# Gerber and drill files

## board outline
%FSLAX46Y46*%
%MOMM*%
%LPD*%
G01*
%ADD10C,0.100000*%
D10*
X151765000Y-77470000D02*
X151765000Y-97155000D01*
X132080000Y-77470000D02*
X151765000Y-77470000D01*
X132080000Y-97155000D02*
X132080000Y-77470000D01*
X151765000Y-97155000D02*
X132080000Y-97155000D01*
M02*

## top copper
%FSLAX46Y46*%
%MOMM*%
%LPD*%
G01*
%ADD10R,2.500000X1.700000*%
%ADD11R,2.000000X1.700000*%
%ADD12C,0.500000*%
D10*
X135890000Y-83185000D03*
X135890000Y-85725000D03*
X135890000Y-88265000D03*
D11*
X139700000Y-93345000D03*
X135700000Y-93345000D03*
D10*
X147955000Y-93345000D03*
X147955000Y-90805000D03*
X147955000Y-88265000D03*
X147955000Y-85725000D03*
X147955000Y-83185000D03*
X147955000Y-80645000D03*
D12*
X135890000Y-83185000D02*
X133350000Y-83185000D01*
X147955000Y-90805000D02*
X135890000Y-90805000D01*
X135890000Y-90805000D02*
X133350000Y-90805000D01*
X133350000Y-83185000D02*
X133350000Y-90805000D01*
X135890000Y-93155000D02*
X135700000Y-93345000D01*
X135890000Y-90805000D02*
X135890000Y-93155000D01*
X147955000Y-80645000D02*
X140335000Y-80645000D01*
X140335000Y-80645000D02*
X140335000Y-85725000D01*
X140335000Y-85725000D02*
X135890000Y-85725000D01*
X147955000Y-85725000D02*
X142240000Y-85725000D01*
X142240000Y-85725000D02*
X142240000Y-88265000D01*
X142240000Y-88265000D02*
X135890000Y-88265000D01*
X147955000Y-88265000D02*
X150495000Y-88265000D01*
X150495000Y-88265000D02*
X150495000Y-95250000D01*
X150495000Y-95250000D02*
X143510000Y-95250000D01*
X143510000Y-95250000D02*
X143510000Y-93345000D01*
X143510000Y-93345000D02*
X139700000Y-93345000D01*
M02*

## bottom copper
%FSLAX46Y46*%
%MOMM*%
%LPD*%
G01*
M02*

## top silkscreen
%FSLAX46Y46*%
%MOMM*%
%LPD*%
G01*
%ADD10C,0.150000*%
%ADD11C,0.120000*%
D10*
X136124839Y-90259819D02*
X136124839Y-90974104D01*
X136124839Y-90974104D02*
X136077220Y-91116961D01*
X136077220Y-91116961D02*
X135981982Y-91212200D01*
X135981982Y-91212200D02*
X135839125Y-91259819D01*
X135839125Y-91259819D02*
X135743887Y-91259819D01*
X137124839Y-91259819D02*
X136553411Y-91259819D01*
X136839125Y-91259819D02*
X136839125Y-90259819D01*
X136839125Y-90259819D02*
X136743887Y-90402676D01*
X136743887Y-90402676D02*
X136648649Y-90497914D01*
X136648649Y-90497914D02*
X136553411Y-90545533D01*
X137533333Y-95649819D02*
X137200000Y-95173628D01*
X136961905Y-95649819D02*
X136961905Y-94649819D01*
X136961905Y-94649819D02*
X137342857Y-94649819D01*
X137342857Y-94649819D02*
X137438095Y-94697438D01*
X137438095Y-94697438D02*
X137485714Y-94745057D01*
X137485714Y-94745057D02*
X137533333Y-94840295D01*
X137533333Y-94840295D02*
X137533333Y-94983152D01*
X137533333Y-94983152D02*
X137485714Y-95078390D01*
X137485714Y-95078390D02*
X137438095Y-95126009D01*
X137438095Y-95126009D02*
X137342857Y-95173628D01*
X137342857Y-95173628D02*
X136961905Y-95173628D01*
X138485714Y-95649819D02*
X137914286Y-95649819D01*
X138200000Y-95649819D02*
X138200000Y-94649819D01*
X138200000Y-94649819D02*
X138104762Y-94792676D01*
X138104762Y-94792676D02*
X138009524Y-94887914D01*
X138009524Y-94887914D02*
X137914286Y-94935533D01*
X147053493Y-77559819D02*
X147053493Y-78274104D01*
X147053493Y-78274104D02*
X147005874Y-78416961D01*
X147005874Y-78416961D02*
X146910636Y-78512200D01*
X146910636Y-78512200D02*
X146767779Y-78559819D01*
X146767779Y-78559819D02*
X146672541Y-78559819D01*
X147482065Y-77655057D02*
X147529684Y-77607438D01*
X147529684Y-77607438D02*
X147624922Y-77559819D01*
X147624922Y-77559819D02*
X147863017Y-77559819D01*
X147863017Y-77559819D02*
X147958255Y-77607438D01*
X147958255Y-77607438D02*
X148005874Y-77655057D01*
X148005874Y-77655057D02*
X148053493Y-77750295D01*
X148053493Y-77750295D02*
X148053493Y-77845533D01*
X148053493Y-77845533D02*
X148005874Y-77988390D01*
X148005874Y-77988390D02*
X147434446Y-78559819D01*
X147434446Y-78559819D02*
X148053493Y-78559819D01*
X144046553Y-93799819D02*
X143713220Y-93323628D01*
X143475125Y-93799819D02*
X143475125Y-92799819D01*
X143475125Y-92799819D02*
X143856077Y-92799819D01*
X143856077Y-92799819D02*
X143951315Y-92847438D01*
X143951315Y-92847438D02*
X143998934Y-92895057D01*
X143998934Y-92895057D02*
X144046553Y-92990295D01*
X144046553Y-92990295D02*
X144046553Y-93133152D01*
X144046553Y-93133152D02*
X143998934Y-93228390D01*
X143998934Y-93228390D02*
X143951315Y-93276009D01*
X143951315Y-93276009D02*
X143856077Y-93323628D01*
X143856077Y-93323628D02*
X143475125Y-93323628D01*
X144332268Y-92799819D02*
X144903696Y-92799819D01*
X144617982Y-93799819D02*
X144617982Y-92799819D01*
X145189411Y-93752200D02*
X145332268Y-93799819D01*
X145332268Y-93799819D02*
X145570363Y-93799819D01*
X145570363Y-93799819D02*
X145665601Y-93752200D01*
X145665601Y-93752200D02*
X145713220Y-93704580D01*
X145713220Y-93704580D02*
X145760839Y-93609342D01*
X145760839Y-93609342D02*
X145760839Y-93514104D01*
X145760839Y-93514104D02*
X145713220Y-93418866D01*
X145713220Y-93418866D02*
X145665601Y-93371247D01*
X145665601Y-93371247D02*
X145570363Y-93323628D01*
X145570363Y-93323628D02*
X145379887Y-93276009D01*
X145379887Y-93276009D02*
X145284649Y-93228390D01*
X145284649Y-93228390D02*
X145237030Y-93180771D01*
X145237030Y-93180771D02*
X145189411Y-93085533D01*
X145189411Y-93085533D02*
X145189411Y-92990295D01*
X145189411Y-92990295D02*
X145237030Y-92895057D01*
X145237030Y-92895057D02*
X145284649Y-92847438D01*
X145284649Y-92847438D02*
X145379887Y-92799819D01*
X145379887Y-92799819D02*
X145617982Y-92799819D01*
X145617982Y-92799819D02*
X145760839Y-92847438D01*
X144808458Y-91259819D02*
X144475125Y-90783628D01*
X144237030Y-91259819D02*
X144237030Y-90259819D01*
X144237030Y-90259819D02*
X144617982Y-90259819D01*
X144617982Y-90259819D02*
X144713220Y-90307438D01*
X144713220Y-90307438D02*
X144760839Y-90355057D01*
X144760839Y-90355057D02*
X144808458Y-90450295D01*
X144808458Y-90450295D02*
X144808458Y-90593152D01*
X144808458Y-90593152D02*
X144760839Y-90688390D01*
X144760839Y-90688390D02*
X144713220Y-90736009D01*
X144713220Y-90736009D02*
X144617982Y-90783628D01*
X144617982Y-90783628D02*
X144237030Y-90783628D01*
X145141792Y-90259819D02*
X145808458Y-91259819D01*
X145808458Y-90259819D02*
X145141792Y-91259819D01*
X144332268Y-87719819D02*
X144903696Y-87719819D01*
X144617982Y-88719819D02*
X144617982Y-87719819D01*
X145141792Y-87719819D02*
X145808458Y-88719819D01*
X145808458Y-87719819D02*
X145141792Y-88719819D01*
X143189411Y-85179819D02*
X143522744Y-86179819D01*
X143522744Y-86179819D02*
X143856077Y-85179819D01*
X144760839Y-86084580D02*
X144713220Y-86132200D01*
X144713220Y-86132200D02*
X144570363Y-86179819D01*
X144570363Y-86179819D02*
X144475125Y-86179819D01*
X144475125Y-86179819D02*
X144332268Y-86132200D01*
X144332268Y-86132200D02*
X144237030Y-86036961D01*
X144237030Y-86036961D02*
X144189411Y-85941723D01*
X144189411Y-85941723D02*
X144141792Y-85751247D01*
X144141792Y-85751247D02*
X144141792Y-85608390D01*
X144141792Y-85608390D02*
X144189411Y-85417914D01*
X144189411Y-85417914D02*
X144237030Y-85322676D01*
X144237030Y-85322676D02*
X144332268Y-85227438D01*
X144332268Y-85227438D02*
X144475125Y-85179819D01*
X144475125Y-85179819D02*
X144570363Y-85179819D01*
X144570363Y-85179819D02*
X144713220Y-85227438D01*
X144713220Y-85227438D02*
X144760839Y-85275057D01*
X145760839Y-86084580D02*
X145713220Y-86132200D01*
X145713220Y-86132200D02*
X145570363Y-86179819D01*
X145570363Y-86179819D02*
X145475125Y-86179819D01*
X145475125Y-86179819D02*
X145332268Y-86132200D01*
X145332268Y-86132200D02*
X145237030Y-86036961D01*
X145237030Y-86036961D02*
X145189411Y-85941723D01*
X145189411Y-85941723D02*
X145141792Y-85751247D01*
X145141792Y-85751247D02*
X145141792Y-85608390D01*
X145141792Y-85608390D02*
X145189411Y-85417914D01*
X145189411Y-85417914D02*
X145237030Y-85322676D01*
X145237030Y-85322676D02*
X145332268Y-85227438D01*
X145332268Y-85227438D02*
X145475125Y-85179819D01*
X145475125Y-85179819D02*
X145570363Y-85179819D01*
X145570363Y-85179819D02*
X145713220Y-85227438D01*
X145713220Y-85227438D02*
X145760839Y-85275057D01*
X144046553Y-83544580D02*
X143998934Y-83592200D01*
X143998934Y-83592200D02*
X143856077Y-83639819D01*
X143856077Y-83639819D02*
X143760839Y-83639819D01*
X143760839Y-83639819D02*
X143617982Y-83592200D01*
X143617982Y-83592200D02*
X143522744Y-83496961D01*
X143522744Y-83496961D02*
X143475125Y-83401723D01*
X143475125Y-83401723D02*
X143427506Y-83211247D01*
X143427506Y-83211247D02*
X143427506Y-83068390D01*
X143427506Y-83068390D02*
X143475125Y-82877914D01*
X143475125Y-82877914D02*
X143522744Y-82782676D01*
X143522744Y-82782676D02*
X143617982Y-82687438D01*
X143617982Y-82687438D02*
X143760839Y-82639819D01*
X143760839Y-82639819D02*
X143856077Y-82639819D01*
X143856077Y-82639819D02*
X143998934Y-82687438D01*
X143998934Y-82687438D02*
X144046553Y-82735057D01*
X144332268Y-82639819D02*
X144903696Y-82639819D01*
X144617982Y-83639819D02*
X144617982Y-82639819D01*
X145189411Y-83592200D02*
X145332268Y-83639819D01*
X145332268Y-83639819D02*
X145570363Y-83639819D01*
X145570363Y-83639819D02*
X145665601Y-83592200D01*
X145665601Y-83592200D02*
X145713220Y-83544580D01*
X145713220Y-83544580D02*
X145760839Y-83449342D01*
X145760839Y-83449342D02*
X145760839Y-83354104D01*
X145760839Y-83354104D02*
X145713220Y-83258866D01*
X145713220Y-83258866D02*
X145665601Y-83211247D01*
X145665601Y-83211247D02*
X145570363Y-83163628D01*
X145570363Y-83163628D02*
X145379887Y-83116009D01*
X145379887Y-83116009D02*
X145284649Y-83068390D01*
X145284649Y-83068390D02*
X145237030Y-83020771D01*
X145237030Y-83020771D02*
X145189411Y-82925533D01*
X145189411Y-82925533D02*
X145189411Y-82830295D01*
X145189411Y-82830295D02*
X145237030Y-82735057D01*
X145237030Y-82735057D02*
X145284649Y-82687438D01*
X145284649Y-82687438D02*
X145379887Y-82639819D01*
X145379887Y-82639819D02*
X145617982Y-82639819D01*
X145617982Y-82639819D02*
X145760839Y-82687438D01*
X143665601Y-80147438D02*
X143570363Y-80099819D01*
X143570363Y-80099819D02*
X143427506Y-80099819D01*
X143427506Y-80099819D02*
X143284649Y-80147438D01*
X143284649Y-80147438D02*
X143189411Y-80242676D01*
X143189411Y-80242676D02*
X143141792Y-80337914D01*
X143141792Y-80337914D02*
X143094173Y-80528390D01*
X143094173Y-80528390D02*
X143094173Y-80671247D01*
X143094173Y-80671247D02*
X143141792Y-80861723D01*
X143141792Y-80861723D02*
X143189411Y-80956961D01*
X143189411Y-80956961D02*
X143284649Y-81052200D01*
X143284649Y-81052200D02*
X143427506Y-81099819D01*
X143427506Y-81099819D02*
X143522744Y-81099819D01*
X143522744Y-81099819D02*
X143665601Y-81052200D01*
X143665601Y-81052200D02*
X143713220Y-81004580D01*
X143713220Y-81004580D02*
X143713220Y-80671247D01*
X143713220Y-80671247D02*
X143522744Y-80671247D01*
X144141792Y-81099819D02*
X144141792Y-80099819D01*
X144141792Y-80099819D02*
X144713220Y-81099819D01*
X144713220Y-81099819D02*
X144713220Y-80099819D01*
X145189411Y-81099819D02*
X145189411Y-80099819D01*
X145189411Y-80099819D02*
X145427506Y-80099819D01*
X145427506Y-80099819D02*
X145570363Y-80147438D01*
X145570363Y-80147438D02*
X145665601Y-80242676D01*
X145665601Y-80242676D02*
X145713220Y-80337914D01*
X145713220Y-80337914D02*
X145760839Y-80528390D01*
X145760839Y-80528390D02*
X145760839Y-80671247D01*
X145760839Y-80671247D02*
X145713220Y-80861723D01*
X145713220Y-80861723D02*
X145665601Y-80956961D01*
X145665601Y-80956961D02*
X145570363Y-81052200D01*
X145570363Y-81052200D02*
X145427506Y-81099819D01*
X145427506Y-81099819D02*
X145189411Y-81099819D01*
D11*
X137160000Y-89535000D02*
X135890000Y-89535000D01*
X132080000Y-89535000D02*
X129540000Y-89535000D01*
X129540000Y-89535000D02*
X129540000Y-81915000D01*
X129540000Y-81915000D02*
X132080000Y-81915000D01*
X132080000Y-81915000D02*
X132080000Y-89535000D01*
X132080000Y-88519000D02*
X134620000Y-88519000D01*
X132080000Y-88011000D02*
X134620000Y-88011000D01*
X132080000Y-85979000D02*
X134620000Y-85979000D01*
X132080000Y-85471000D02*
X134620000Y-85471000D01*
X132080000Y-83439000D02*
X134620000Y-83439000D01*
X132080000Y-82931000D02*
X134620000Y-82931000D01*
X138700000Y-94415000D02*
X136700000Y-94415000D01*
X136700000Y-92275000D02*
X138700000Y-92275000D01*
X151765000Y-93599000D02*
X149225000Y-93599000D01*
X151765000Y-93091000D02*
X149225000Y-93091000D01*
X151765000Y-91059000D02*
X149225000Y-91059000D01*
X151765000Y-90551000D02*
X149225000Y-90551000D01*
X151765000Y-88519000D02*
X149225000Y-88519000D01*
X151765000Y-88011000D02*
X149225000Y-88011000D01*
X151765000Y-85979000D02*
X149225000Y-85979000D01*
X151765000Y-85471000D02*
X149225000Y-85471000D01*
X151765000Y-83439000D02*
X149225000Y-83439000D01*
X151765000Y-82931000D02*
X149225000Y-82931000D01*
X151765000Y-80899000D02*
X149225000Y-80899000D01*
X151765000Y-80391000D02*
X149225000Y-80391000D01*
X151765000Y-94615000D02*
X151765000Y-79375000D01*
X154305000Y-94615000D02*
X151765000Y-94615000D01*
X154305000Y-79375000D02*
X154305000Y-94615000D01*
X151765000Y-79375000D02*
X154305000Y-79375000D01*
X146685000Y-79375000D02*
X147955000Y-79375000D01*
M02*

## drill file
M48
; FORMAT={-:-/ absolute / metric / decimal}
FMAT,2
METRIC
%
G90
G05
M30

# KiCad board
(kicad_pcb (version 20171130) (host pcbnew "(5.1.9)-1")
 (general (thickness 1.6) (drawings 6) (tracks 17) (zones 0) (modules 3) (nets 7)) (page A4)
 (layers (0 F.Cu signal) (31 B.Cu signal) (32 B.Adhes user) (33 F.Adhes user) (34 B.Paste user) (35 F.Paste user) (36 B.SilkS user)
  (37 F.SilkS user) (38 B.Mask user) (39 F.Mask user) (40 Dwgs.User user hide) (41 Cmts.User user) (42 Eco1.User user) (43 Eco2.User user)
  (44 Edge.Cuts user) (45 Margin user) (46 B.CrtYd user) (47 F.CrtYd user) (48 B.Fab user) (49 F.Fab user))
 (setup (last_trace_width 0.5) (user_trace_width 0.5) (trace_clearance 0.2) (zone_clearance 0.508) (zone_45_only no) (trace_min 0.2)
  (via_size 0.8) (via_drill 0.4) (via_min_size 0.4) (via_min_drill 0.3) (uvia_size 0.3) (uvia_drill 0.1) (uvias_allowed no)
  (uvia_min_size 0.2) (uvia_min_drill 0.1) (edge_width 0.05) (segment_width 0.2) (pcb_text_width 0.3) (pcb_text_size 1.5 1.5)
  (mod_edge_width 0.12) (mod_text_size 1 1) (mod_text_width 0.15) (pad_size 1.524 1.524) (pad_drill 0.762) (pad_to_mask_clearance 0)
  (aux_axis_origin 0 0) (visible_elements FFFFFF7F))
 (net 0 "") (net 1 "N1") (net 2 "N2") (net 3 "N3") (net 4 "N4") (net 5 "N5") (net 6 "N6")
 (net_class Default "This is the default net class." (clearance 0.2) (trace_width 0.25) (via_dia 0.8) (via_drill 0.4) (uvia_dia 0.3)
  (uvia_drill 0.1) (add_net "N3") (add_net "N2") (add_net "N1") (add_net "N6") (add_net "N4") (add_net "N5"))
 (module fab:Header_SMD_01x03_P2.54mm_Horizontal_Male (layer F.Cu) (at 135.89 88.265 180)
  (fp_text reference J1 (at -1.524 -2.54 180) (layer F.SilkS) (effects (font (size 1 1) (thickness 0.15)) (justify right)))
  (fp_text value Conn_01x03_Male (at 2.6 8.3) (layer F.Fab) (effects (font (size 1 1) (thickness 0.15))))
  (fp_line (start -1.27 -1.27) (end 0 -1.27) (layer F.SilkS) (width 0.12))
  (fp_line (start 3.81 -1.27) (end 6.35 -1.27) (layer F.SilkS) (width 0.12))
  (fp_line (start 6.35 -1.27) (end 6.35 6.35) (layer F.SilkS) (width 0.12))
  (fp_line (start 6.35 6.35) (end 3.81 6.35) (layer F.SilkS) (width 0.12))
  (fp_line (start 3.81 6.35) (end 3.81 -1.27) (layer F.SilkS) (width 0.12))
  (fp_line (start 3.81 -0.254) (end 1.27 -0.254) (layer F.SilkS) (width 0.12))
  (fp_line (start 3.81 0.254) (end 1.27 0.254) (layer F.SilkS) (width 0.12))
  (fp_line (start 3.81 2.286) (end 1.27 2.286) (layer F.SilkS) (width 0.12))
  (fp_line (start 3.81 2.794) (end 1.27 2.794) (layer F.SilkS) (width 0.12))
  (fp_line (start 3.81 4.826) (end 1.27 4.826) (layer F.SilkS) (width 0.12))
  (fp_line (start 3.81 5.334) (end 1.27 5.334) (layer F.SilkS) (width 0.12))
  (pad 3 smd rect (at 0 5.08 180) (size 2.5 1.7) (layers F.Cu F.Paste F.Mask) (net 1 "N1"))
  (pad 2 smd rect (at 0 2.54 180) (size 2.5 1.7) (layers F.Cu F.Paste F.Mask) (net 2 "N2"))
  (pad 1 smd rect (at 0 0 180) (size 2.5 1.7) (layers F.Cu F.Paste F.Mask) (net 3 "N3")))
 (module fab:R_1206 (layer F.Cu) (at 137.7 93.345 180)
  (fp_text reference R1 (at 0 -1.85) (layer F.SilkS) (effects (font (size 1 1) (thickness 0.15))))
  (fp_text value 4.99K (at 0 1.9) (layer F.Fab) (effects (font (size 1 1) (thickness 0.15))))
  (fp_line (start -1 -1.07) (end 1 -1.07) (layer F.SilkS) (width 0.12))
  (fp_line (start 1 1.07) (end -1 1.07) (layer F.SilkS) (width 0.12))
  (pad 1 smd rect (at -2 0 180) (size 2 1.7) (layers F.Cu F.Paste F.Mask) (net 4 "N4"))
  (pad 2 smd rect (at 2 0 180) (size 2 1.7) (layers F.Cu F.Paste F.Mask) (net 1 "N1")))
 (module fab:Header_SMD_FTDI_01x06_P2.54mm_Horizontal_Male (layer F.Cu) (at 147.955 80.645)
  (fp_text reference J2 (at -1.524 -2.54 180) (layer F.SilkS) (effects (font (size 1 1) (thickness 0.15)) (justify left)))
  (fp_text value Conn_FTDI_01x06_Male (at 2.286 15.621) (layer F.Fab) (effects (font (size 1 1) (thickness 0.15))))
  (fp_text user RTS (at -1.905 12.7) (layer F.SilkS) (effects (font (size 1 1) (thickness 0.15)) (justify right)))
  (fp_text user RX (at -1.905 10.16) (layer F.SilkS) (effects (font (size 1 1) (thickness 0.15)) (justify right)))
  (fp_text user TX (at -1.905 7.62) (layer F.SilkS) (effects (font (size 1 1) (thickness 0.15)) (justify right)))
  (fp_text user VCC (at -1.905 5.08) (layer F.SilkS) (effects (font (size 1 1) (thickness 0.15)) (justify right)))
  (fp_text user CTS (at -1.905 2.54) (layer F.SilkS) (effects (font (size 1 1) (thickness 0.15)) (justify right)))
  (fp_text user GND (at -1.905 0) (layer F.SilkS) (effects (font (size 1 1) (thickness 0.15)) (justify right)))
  (fp_line (start 3.81 12.954) (end 1.27 12.954) (layer F.SilkS) (width 0.12))
  (fp_line (start 3.81 12.446) (end 1.27 12.446) (layer F.SilkS) (width 0.12))
  (fp_line (start 3.81 10.414) (end 1.27 10.414) (layer F.SilkS) (width 0.12))
  (fp_line (start 3.81 9.906) (end 1.27 9.906) (layer F.SilkS) (width 0.12))
  (fp_line (start 3.81 7.874) (end 1.27 7.874) (layer F.SilkS) (width 0.12))
  (fp_line (start 3.81 7.366) (end 1.27 7.366) (layer F.SilkS) (width 0.12))
  (fp_line (start 3.81 5.334) (end 1.27 5.334) (layer F.SilkS) (width 0.12))
  (fp_line (start 3.81 4.826) (end 1.27 4.826) (layer F.SilkS) (width 0.12))
  (fp_line (start 3.81 2.794) (end 1.27 2.794) (layer F.SilkS) (width 0.12))
  (fp_line (start 3.81 2.286) (end 1.27 2.286) (layer F.SilkS) (width 0.12))
  (fp_line (start 3.81 0.254) (end 1.27 0.254) (layer F.SilkS) (width 0.12))
  (fp_line (start 3.81 -0.254) (end 1.27 -0.254) (layer F.SilkS) (width 0.12))
  (fp_line (start 3.81 13.97) (end 3.81 -1.27) (layer F.SilkS) (width 0.12))
  (fp_line (start 6.35 13.97) (end 3.81 13.97) (layer F.SilkS) (width 0.12))
  (fp_line (start 6.35 -1.27) (end 6.35 13.97) (layer F.SilkS) (width 0.12))
  (fp_line (start 3.81 -1.27) (end 6.35 -1.27) (layer F.SilkS) (width 0.12))
  (fp_line (start -1.27 -1.27) (end 0 -1.27) (layer F.SilkS) (width 0.12))
  (pad 6 smd rect (at 0 12.7) (size 2.5 1.7) (layers F.Cu F.Paste F.Mask) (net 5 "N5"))
  (pad 5 smd rect (at 0 10.16) (size 2.5 1.7) (layers F.Cu F.Paste F.Mask) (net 1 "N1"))
  (pad 4 smd rect (at 0 7.62) (size 2.5 1.7) (layers F.Cu F.Paste F.Mask) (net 4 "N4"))
  (pad 3 smd rect (at 0 5.08) (size 2.5 1.7) (layers F.Cu F.Paste F.Mask) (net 3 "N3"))
  (pad 2 smd rect (at 0 2.54) (size 2.5 1.7) (layers F.Cu F.Paste F.Mask) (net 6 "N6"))
  (pad 1 smd rect (at 0 0) (size 2.5 1.7) (layers F.Cu F.Paste F.Mask) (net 2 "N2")))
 (gr_line (start 151.765 77.47) (end 151.765 97.155) (layer Edge.Cuts) (width 0.1))
 (gr_line (start 132.08 77.47) (end 151.765 77.47) (layer Edge.Cuts) (width 0.1))
 (gr_line (start 132.08 97.155) (end 132.08 77.47) (layer Edge.Cuts) (width 0.1))
 (gr_line (start 151.765 97.155) (end 132.08 97.155) (layer Edge.Cuts) (width 0.1))
 (segment (start 135.89 83.185) (end 133.35 83.185) (width 0.5) (layer F.Cu) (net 1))
 (segment (start 147.955 90.805) (end 135.89 90.805) (width 0.5) (layer F.Cu) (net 1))
 (segment (start 135.89 90.805) (end 133.35 90.805) (width 0.5) (layer F.Cu) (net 1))
 (segment (start 133.35 83.185) (end 133.35 90.805) (width 0.5) (layer F.Cu) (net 1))
 (segment (start 135.89 93.155) (end 135.7 93.345) (width 0.5) (layer F.Cu) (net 1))
 (segment (start 135.89 90.805) (end 135.89 93.155) (width 0.5) (layer F.Cu) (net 1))
 (segment (start 147.955 80.645) (end 140.335 80.645) (width 0.5) (layer F.Cu) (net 2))
 (segment (start 140.335 80.645) (end 140.335 85.725) (width 0.5) (layer F.Cu) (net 2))
 (segment (start 140.335 85.725) (end 135.89 85.725) (width 0.5) (layer F.Cu) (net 2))
 (segment (start 147.955 85.725) (end 142.24 85.725) (width 0.5) (layer F.Cu) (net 3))
 (segment (start 142.24 85.725) (end 142.24 88.265) (width 0.5) (layer F.Cu) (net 3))
 (segment (start 142.24 88.265) (end 135.89 88.265) (width 0.5) (layer F.Cu) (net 3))
 (segment (start 147.955 88.265) (end 150.495 88.265) (width 0.5) (layer F.Cu) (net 4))
 (segment (start 150.495 88.265) (end 150.495 95.25) (width 0.5) (layer F.Cu) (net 4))
 (segment (start 150.495 95.25) (end 143.51 95.25) (width 0.5) (layer F.Cu) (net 4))
 (segment (start 143.51 95.25) (end 143.51 93.345) (width 0.5) (layer F.Cu) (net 4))
 (segment (start 143.51 93.345) (end 139.7 93.345) (width 0.5) (layer F.Cu) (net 4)))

